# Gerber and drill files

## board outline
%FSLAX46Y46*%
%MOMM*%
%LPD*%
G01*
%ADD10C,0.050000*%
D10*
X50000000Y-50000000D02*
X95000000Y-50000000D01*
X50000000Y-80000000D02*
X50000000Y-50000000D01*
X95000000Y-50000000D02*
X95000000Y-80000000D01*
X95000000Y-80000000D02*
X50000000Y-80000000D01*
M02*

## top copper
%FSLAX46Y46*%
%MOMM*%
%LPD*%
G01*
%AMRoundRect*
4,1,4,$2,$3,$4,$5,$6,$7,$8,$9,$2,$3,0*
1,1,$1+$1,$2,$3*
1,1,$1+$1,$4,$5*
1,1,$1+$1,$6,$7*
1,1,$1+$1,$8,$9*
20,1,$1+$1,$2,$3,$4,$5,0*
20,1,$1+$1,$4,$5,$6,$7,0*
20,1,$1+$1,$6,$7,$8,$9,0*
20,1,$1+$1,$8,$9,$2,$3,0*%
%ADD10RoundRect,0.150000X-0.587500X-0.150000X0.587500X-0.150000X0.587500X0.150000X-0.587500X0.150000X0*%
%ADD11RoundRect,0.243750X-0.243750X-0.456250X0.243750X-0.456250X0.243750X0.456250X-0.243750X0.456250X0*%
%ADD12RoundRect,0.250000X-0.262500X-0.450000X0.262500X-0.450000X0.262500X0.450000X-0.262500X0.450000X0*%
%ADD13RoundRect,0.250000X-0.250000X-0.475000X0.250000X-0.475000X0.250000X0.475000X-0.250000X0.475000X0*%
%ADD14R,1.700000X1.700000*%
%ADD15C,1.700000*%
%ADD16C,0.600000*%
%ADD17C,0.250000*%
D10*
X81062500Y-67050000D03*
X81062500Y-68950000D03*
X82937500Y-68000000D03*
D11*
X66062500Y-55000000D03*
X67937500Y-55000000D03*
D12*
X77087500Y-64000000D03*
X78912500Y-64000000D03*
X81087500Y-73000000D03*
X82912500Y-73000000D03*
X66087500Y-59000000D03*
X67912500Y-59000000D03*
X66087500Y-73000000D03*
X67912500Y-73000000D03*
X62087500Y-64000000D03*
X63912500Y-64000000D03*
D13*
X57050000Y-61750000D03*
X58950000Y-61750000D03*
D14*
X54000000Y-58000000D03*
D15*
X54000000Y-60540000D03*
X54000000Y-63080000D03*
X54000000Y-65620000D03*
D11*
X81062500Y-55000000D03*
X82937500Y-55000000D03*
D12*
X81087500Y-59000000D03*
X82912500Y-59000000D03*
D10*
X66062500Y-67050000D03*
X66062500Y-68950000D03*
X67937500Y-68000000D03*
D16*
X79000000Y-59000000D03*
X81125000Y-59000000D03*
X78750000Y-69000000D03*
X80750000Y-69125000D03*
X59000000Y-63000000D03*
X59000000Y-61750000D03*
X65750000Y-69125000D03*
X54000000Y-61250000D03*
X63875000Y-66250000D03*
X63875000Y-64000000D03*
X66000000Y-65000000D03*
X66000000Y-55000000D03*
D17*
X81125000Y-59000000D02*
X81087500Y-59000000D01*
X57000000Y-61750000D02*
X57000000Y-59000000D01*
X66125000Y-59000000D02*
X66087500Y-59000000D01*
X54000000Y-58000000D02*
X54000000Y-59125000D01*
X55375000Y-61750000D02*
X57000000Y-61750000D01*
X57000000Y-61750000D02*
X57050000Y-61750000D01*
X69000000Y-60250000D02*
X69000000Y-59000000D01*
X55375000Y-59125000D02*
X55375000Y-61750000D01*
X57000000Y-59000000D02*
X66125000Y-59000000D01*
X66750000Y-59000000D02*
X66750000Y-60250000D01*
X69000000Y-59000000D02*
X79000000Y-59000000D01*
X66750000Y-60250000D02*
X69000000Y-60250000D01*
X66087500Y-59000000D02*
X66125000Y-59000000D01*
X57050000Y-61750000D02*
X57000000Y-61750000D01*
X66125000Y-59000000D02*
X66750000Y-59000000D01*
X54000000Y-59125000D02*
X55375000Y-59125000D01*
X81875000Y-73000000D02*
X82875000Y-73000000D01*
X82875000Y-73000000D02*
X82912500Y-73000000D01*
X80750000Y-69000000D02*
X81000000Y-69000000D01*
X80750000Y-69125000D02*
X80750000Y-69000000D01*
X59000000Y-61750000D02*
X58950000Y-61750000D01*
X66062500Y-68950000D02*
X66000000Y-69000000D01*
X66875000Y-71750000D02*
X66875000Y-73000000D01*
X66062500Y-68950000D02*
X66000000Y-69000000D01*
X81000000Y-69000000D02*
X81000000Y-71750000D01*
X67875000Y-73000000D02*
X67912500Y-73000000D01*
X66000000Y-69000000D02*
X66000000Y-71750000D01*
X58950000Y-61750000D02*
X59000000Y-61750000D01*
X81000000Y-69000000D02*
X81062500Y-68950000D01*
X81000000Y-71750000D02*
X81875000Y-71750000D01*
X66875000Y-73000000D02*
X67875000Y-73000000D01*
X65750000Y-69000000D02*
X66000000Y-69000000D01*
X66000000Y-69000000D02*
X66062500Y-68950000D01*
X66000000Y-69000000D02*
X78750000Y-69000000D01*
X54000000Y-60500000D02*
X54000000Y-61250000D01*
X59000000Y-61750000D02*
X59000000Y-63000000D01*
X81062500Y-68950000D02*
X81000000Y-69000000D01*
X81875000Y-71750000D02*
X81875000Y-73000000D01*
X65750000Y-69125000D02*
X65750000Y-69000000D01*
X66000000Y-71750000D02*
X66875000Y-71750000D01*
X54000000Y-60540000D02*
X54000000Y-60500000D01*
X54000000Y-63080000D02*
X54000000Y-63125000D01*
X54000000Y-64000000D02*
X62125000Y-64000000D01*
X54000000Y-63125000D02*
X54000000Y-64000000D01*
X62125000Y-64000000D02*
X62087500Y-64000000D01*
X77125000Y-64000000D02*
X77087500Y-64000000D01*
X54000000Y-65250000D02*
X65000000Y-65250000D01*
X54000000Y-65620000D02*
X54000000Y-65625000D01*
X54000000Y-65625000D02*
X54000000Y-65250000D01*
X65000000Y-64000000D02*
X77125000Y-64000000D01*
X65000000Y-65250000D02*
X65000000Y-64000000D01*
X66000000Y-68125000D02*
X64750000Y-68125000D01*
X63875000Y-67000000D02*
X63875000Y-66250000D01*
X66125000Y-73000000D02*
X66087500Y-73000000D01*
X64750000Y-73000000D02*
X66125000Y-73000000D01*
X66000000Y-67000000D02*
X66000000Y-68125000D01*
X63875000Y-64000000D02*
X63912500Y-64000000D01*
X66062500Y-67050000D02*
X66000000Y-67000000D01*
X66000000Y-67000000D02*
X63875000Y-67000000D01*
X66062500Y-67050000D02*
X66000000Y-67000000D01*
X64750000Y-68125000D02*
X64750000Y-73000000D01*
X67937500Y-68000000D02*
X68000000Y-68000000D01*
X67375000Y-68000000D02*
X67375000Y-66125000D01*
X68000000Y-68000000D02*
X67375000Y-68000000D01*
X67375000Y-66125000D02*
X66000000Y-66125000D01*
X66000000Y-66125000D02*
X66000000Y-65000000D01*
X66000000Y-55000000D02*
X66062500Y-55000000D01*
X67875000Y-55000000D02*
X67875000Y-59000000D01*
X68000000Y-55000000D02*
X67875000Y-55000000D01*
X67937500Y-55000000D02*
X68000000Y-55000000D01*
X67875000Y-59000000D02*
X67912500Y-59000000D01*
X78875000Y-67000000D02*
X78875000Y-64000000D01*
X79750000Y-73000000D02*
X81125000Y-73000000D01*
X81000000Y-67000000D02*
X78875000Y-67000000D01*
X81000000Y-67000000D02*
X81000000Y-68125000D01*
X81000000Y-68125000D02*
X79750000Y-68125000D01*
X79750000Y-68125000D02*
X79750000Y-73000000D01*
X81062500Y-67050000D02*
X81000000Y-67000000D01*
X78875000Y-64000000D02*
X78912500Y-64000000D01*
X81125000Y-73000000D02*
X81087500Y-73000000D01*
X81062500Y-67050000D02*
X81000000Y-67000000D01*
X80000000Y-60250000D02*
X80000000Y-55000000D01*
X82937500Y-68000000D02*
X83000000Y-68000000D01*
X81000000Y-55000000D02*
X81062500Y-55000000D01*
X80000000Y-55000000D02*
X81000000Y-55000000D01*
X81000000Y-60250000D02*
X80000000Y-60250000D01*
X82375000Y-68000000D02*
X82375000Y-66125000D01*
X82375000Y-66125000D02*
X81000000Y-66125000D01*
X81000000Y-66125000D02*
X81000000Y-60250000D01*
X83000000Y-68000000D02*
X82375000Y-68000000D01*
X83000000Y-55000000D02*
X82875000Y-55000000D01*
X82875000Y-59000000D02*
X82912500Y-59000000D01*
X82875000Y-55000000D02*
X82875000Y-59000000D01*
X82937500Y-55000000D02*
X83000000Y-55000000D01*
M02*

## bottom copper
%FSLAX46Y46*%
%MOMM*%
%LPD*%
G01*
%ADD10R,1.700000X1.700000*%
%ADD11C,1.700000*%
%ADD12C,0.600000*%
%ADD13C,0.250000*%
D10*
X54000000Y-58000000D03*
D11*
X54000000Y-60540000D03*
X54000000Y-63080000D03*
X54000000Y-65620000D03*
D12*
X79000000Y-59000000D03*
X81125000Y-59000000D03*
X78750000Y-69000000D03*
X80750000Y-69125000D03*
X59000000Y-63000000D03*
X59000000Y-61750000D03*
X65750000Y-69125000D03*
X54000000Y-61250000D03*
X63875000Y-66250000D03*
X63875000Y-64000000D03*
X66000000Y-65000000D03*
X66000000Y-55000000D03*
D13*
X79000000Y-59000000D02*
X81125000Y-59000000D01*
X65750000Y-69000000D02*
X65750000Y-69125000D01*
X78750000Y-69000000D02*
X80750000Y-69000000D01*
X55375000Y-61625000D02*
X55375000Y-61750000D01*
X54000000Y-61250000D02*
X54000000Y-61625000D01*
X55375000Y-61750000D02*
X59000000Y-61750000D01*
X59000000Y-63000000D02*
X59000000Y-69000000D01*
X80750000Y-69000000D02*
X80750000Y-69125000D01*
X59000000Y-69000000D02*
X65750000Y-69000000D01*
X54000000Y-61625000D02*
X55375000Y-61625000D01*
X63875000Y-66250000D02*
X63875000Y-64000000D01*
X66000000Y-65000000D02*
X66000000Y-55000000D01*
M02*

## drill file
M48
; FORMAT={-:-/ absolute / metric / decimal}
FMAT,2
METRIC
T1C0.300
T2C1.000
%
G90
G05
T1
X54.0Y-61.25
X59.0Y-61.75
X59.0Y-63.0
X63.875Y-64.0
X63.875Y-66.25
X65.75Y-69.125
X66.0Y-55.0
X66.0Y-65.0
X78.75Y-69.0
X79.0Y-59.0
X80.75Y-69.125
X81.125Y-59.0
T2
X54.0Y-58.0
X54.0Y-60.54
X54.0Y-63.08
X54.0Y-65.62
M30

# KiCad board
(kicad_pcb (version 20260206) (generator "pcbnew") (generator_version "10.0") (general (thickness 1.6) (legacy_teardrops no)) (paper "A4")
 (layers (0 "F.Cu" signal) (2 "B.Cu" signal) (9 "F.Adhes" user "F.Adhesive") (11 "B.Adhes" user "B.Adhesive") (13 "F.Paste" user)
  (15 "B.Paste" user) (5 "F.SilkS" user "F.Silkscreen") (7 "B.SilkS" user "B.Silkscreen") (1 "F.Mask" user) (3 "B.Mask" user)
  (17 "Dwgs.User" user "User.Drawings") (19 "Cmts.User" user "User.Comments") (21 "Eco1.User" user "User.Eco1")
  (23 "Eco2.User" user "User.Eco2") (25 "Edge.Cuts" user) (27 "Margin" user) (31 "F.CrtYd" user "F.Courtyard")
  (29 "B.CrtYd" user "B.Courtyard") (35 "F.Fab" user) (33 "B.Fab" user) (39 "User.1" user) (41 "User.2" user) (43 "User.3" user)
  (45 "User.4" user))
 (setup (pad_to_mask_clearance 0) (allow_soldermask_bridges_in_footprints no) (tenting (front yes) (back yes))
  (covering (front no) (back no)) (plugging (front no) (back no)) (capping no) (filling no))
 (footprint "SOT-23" (layer "F.Cu") (at 82 68)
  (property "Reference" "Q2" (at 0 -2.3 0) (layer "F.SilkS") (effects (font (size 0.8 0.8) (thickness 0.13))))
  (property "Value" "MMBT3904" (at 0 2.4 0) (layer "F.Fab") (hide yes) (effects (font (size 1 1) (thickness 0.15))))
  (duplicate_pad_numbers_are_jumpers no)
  (pad "1" smd roundrect (at -0.9375 -0.95) (size 1.475 0.6) (layers "F.Cu" "F.Mask" "F.Paste") (roundrect_rratio 0.25) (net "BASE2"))
  (pad "2" smd roundrect (at -0.9375 0.95) (size 1.475 0.6) (layers "F.Cu" "F.Mask" "F.Paste") (roundrect_rratio 0.25) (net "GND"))
  (pad "3" smd roundrect (at 0.9375 0) (size 1.475 0.6) (layers "F.Cu" "F.Mask" "F.Paste") (roundrect_rratio 0.25) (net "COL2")))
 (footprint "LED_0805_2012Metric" (layer "F.Cu") (at 67 55)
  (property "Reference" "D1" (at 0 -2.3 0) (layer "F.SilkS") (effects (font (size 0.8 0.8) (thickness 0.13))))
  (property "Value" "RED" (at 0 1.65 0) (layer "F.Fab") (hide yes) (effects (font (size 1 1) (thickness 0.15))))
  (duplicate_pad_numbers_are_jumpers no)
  (pad "1" smd roundrect (at -0.9375 0) (size 0.975 1.4) (layers "F.Cu" "F.Mask" "F.Paste") (roundrect_rratio 0.25) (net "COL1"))
  (pad "2" smd roundrect (at 0.9375 0) (size 0.975 1.4) (layers "F.Cu" "F.Mask" "F.Paste") (roundrect_rratio 0.25) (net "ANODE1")))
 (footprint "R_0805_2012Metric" (layer "F.Cu") (at 78 64)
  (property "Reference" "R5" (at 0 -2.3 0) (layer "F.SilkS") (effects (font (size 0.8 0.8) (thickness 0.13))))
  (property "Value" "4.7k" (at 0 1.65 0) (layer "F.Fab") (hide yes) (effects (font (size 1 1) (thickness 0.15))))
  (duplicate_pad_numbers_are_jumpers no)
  (pad "1" smd roundrect (at -0.9125 0) (size 1.025 1.4) (layers "F.Cu" "F.Mask" "F.Paste") (roundrect_rratio 0.243902) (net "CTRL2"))
  (pad "2" smd roundrect (at 0.9125 0) (size 1.025 1.4) (layers "F.Cu" "F.Mask" "F.Paste") (roundrect_rratio 0.243902) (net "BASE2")))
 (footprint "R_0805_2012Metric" (layer "F.Cu") (at 82 73)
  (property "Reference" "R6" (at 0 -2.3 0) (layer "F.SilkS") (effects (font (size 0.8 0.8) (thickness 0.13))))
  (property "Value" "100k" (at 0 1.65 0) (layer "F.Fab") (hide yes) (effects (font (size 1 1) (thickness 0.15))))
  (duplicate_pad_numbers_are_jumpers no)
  (pad "1" smd roundrect (at -0.9125 0) (size 1.025 1.4) (layers "F.Cu" "F.Mask" "F.Paste") (roundrect_rratio 0.243902) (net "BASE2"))
  (pad "2" smd roundrect (at 0.9125 0) (size 1.025 1.4) (layers "F.Cu" "F.Mask" "F.Paste") (roundrect_rratio 0.243902) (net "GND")))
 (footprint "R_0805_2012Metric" (layer "F.Cu") (at 67 59)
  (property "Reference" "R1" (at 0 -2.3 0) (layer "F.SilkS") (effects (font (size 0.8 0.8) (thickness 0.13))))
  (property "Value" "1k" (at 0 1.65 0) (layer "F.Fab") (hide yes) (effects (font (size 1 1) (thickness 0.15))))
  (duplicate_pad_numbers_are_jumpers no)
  (pad "1" smd roundrect (at -0.9125 0) (size 1.025 1.4) (layers "F.Cu" "F.Mask" "F.Paste") (roundrect_rratio 0.243902) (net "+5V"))
  (pad "2" smd roundrect (at 0.9125 0) (size 1.025 1.4) (layers "F.Cu" "F.Mask" "F.Paste") (roundrect_rratio 0.243902) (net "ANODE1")))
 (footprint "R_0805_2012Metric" (layer "F.Cu") (at 67 73)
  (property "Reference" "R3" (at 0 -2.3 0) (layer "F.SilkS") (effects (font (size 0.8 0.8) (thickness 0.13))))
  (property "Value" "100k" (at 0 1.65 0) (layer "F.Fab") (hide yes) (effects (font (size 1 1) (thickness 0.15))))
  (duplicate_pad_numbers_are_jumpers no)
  (pad "1" smd roundrect (at -0.9125 0) (size 1.025 1.4) (layers "F.Cu" "F.Mask" "F.Paste") (roundrect_rratio 0.243902) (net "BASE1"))
  (pad "2" smd roundrect (at 0.9125 0) (size 1.025 1.4) (layers "F.Cu" "F.Mask" "F.Paste") (roundrect_rratio 0.243902) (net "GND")))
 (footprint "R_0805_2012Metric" (layer "F.Cu") (at 63 64)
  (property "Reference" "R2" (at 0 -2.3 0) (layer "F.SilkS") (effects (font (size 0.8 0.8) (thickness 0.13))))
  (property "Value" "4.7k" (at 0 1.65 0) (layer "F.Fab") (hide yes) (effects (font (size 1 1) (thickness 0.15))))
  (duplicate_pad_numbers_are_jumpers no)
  (pad "1" smd roundrect (at -0.9125 0) (size 1.025 1.4) (layers "F.Cu" "F.Mask" "F.Paste") (roundrect_rratio 0.243902) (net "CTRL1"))
  (pad "2" smd roundrect (at 0.9125 0) (size 1.025 1.4) (layers "F.Cu" "F.Mask" "F.Paste") (roundrect_rratio 0.243902) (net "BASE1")))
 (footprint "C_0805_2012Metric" (layer "F.Cu") (at 58 61.75)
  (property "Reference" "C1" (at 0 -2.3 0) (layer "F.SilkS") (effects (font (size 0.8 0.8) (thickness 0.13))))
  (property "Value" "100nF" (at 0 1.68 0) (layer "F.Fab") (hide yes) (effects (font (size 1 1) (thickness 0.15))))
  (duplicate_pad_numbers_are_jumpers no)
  (pad "1" smd roundrect (at -0.95 0) (size 1 1.45) (layers "F.Cu" "F.Mask" "F.Paste") (roundrect_rratio 0.25) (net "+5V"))
  (pad "2" smd roundrect (at 0.95 0) (size 1 1.45) (layers "F.Cu" "F.Mask" "F.Paste") (roundrect_rratio 0.25) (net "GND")))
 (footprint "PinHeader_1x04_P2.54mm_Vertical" (layer "F.Cu") (at 54 58)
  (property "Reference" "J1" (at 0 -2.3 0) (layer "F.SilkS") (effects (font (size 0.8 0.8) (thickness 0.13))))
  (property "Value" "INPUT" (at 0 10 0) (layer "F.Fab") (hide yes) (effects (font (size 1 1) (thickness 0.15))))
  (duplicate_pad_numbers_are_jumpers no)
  (pad "1" thru_hole rect (at 0 0) (size 1.7 1.7) (drill 1) (layers "*.Cu" "*.Mask") (remove_unused_layers no) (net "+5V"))
  (pad "2" thru_hole circle (at 0 2.54) (size 1.7 1.7) (drill 1) (layers "*.Cu" "*.Mask") (remove_unused_layers no) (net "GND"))
  (pad "3" thru_hole circle (at 0 5.08) (size 1.7 1.7) (drill 1) (layers "*.Cu" "*.Mask") (remove_unused_layers no) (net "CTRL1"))
  (pad "4" thru_hole circle (at 0 7.62) (size 1.7 1.7) (drill 1) (layers "*.Cu" "*.Mask") (remove_unused_layers no) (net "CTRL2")))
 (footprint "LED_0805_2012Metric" (layer "F.Cu") (at 82 55)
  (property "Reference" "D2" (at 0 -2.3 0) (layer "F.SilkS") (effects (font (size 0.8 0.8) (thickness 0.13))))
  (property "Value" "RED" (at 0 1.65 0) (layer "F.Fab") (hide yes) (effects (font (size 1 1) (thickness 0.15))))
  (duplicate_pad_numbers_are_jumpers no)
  (pad "1" smd roundrect (at -0.9375 0) (size 0.975 1.4) (layers "F.Cu" "F.Mask" "F.Paste") (roundrect_rratio 0.25) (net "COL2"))
  (pad "2" smd roundrect (at 0.9375 0) (size 0.975 1.4) (layers "F.Cu" "F.Mask" "F.Paste") (roundrect_rratio 0.25) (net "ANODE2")))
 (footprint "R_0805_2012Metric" (layer "F.Cu") (at 82 59)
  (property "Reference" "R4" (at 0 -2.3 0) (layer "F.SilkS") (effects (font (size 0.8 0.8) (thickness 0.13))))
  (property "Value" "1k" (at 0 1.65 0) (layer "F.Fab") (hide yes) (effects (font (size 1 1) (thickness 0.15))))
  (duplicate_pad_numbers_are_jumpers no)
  (pad "1" smd roundrect (at -0.9125 0) (size 1.025 1.4) (layers "F.Cu" "F.Mask" "F.Paste") (roundrect_rratio 0.243902) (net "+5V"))
  (pad "2" smd roundrect (at 0.9125 0) (size 1.025 1.4) (layers "F.Cu" "F.Mask" "F.Paste") (roundrect_rratio 0.243902) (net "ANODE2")))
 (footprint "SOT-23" (layer "F.Cu") (at 67 68)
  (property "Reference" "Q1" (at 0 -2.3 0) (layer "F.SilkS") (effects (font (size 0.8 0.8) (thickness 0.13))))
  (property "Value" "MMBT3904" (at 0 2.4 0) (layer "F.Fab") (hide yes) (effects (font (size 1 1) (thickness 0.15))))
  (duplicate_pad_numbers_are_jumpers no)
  (pad "1" smd roundrect (at -0.9375 -0.95) (size 1.475 0.6) (layers "F.Cu" "F.Mask" "F.Paste") (roundrect_rratio 0.25) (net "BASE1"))
  (pad "2" smd roundrect (at -0.9375 0.95) (size 1.475 0.6) (layers "F.Cu" "F.Mask" "F.Paste") (roundrect_rratio 0.25) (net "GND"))
  (pad "3" smd roundrect (at 0.9375 0) (size 1.475 0.6) (layers "F.Cu" "F.Mask" "F.Paste") (roundrect_rratio 0.25) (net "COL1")))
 (gr_line (start 50 50) (end 95 50) (stroke (width 0.05) (type default)) (layer "Edge.Cuts"))
 (gr_line (start 50 80) (end 50 50) (stroke (width 0.05) (type default)) (layer "Edge.Cuts"))
 (gr_line (start 95 50) (end 95 80) (stroke (width 0.05) (type default)) (layer "Edge.Cuts"))
 (gr_line (start 95 80) (end 50 80) (stroke (width 0.05) (type default)) (layer "Edge.Cuts"))
 (segment (start 81.125 59) (end 81.0875 59) (width 0.25) (layer "F.Cu") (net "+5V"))
 (segment (start 57 61.75) (end 57 59) (width 0.25) (layer "F.Cu") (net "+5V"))
 (segment (start 66.125 59) (end 66.0875 59) (width 0.25) (layer "F.Cu") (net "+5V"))
 (segment (start 54 58) (end 54 59.125) (width 0.25) (layer "F.Cu") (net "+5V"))
 (segment (start 55.375 61.75) (end 57 61.75) (width 0.25) (layer "F.Cu") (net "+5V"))
 (segment (start 57 61.75) (end 57.05 61.75) (width 0.25) (layer "F.Cu") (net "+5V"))
 (segment (start 69 60.25) (end 69 59) (width 0.25) (layer "F.Cu") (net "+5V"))
 (segment (start 55.375 59.125) (end 55.375 61.75) (width 0.25) (layer "F.Cu") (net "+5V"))
 (segment (start 57 59) (end 66.125 59) (width 0.25) (layer "F.Cu") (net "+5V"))
 (segment (start 66.75 59) (end 66.75 60.25) (width 0.25) (layer "F.Cu") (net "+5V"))
 (segment (start 69 59) (end 79 59) (width 0.25) (layer "F.Cu") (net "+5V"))
 (segment (start 66.75 60.25) (end 69 60.25) (width 0.25) (layer "F.Cu") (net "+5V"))
 (segment (start 66.0875 59) (end 66.125 59) (width 0.25) (layer "F.Cu") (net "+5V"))
 (segment (start 57.05 61.75) (end 57 61.75) (width 0.25) (layer "F.Cu") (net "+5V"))
 (segment (start 66.125 59) (end 66.75 59) (width 0.25) (layer "F.Cu") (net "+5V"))
 (segment (start 54 59.125) (end 55.375 59.125) (width 0.25) (layer "F.Cu") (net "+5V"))
 (via (at 79 59) (size 0.6) (drill 0.3) (layers "F.Cu" "B.Cu") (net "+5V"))
 (via (at 81.125 59) (size 0.6) (drill 0.3) (layers "F.Cu" "B.Cu") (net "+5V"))
 (segment (start 79 59) (end 81.125 59) (width 0.25) (layer "B.Cu") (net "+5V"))
 (segment (start 81.875 73) (end 82.875 73) (width 0.25) (layer "F.Cu") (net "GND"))
 (segment (start 82.875 73) (end 82.9125 73) (width 0.25) (layer "F.Cu") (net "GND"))
 (segment (start 80.75 69) (end 81 69) (width 0.25) (layer "F.Cu") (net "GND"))
 (segment (start 80.75 69.125) (end 80.75 69) (width 0.25) (layer "F.Cu") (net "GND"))
 (segment (start 59 61.75) (end 58.95 61.75) (width 0.25) (layer "F.Cu") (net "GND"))
 (segment (start 66.0625 68.95) (end 66 69) (width 0.25) (layer "F.Cu") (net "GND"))
 (segment (start 66.875 71.75) (end 66.875 73) (width 0.25) (layer "F.Cu") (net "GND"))
 (segment (start 66.0625 68.95) (end 66 69) (width 0.25) (layer "F.Cu") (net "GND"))
 (segment (start 81 69) (end 81 71.75) (width 0.25) (layer "F.Cu") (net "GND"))
 (segment (start 67.875 73) (end 67.9125 73) (width 0.25) (layer "F.Cu") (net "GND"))
 (segment (start 66 69) (end 66 71.75) (width 0.25) (layer "F.Cu") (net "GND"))
 (segment (start 58.95 61.75) (end 59 61.75) (width 0.25) (layer "F.Cu") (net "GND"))
 (segment (start 81 69) (end 81.0625 68.95) (width 0.25) (layer "F.Cu") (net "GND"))
 (segment (start 81 71.75) (end 81.875 71.75) (width 0.25) (layer "F.Cu") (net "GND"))
 (segment (start 66.875 73) (end 67.875 73) (width 0.25) (layer "F.Cu") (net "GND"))
 (segment (start 65.75 69) (end 66 69) (width 0.25) (layer "F.Cu") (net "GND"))
 (segment (start 66 69) (end 66.0625 68.95) (width 0.25) (layer "F.Cu") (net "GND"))
 (segment (start 66 69) (end 78.75 69) (width 0.25) (layer "F.Cu") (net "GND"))
 (segment (start 54 60.5) (end 54 61.25) (width 0.25) (layer "F.Cu") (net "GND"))
 (segment (start 59 61.75) (end 59 63) (width 0.25) (layer "F.Cu") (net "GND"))
 (segment (start 81.0625 68.95) (end 81 69) (width 0.25) (layer "F.Cu") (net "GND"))
 (segment (start 81.875 71.75) (end 81.875 73) (width 0.25) (layer "F.Cu") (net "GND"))
 (segment (start 65.75 69.125) (end 65.75 69) (width 0.25) (layer "F.Cu") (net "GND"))
 (segment (start 66 71.75) (end 66.875 71.75) (width 0.25) (layer "F.Cu") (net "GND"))
 (segment (start 54 60.54) (end 54 60.5) (width 0.25) (layer "F.Cu") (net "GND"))
 (via (at 78.75 69) (size 0.6) (drill 0.3) (layers "F.Cu" "B.Cu") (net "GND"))
 (via (at 80.75 69.125) (size 0.6) (drill 0.3) (layers "F.Cu" "B.Cu") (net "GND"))
 (via (at 59 63) (size 0.6) (drill 0.3) (layers "F.Cu" "B.Cu") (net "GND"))
 (via (at 59 61.75) (size 0.6) (drill 0.3) (layers "F.Cu" "B.Cu") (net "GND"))
 (via (at 65.75 69.125) (size 0.6) (drill 0.3) (layers "F.Cu" "B.Cu") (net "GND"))
 (via (at 54 61.25) (size 0.6) (drill 0.3) (layers "F.Cu" "B.Cu") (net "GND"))
 (segment (start 65.75 69) (end 65.75 69.125) (width 0.25) (layer "B.Cu") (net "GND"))
 (segment (start 78.75 69) (end 80.75 69) (width 0.25) (layer "B.Cu") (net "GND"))
 (segment (start 55.375 61.625) (end 55.375 61.75) (width 0.25) (layer "B.Cu") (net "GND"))
 (segment (start 54 61.25) (end 54 61.625) (width 0.25) (layer "B.Cu") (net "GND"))
 (segment (start 55.375 61.75) (end 59 61.75) (width 0.25) (layer "B.Cu") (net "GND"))
 (segment (start 59 63) (end 59 69) (width 0.25) (layer "B.Cu") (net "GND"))
 (segment (start 80.75 69) (end 80.75 69.125) (width 0.25) (layer "B.Cu") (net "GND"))
 (segment (start 59 69) (end 65.75 69) (width 0.25) (layer "B.Cu") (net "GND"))
 (segment (start 54 61.625) (end 55.375 61.625) (width 0.25) (layer "B.Cu") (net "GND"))
 (segment (start 54 63.08) (end 54 63.125) (width 0.25) (layer "F.Cu") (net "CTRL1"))
 (segment (start 54 64) (end 62.125 64) (width 0.25) (layer "F.Cu") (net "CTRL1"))
 (segment (start 54 63.125) (end 54 64) (width 0.25) (layer "F.Cu") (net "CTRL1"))
 (segment (start 62.125 64) (end 62.0875 64) (width 0.25) (layer "F.Cu") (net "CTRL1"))
 (segment (start 77.125 64) (end 77.0875 64) (width 0.25) (layer "F.Cu") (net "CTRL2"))
 (segment (start 54 65.25) (end 65 65.25) (width 0.25) (layer "F.Cu") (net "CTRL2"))
 (segment (start 54 65.62) (end 54 65.625) (width 0.25) (layer "F.Cu") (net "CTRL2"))
 (segment (start 54 65.625) (end 54 65.25) (width 0.25) (layer "F.Cu") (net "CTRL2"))
 (segment (start 65 64) (end 77.125 64) (width 0.25) (layer "F.Cu") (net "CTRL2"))
 (segment (start 65 65.25) (end 65 64) (width 0.25) (layer "F.Cu") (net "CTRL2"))
 (segment (start 66 68.125) (end 64.75 68.125) (width 0.25) (layer "F.Cu") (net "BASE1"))
 (segment (start 63.875 67) (end 63.875 66.25) (width 0.25) (layer "F.Cu") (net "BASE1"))
 (segment (start 66.125 73) (end 66.0875 73) (width 0.25) (layer "F.Cu") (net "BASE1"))
 (segment (start 64.75 73) (end 66.125 73) (width 0.25) (layer "F.Cu") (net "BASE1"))
 (segment (start 66 67) (end 66 68.125) (width 0.25) (layer "F.Cu") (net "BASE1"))
 (segment (start 63.875 64) (end 63.9125 64) (width 0.25) (layer "F.Cu") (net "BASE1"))
 (segment (start 66.0625 67.05) (end 66 67) (width 0.25) (layer "F.Cu") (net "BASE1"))
 (segment (start 66 67) (end 63.875 67) (width 0.25) (layer "F.Cu") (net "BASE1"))
 (segment (start 66.0625 67.05) (end 66 67) (width 0.25) (layer "F.Cu") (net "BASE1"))
 (segment (start 64.75 68.125) (end 64.75 73) (width 0.25) (layer "F.Cu") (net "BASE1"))
 (via (at 63.875 66.25) (size 0.6) (drill 0.3) (layers "F.Cu" "B.Cu") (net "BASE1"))
 (via (at 63.875 64) (size 0.6) (drill 0.3) (layers "F.Cu" "B.Cu") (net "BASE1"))
 (segment (start 63.875 66.25) (end 63.875 64) (width 0.25) (layer "B.Cu") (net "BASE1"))
 (segment (start 67.9375 68) (end 68 68) (width 0.25) (layer "F.Cu") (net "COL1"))
 (segment (start 67.375 68) (end 67.375 66.125) (width 0.25) (layer "F.Cu") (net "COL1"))
 (segment (start 68 68) (end 67.375 68) (width 0.25) (layer "F.Cu") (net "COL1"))
 (segment (start 67.375 66.125) (end 66 66.125) (width 0.25) (layer "F.Cu") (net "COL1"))
 (segment (start 66 66.125) (end 66 65) (width 0.25) (layer "F.Cu") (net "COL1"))
 (segment (start 66 55) (end 66.0625 55) (width 0.25) (layer "F.Cu") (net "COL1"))
 (via (at 66 65) (size 0.6) (drill 0.3) (layers "F.Cu" "B.Cu") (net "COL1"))
 (via (at 66 55) (size 0.6) (drill 0.3) (layers "F.Cu" "B.Cu") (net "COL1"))
 (segment (start 66 65) (end 66 55) (width 0.25) (layer "B.Cu") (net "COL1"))
 (segment (start 67.875 55) (end 67.875 59) (width 0.25) (layer "F.Cu") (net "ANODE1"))
 (segment (start 68 55) (end 67.875 55) (width 0.25) (layer "F.Cu") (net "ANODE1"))
 (segment (start 67.9375 55) (end 68 55) (width 0.25) (layer "F.Cu") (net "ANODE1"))
 (segment (start 67.875 59) (end 67.9125 59) (width 0.25) (layer "F.Cu") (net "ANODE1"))
 (segment (start 78.875 67) (end 78.875 64) (width 0.25) (layer "F.Cu") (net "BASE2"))
 (segment (start 79.75 73) (end 81.125 73) (width 0.25) (layer "F.Cu") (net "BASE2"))
 (segment (start 81 67) (end 78.875 67) (width 0.25) (layer "F.Cu") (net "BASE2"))
 (segment (start 81 67) (end 81 68.125) (width 0.25) (layer "F.Cu") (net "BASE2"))
 (segment (start 81 68.125) (end 79.75 68.125) (width 0.25) (layer "F.Cu") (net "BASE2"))
 (segment (start 79.75 68.125) (end 79.75 73) (width 0.25) (layer "F.Cu") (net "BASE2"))
 (segment (start 81.0625 67.05) (end 81 67) (width 0.25) (layer "F.Cu") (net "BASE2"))
 (segment (start 78.875 64) (end 78.9125 64) (width 0.25) (layer "F.Cu") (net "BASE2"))
 (segment (start 81.125 73) (end 81.0875 73) (width 0.25) (layer "F.Cu") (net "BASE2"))
 (segment (start 81.0625 67.05) (end 81 67) (width 0.25) (layer "F.Cu") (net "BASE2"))
 (segment (start 80 60.25) (end 80 55) (width 0.25) (layer "F.Cu") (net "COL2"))
 (segment (start 82.9375 68) (end 83 68) (width 0.25) (layer "F.Cu") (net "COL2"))
 (segment (start 81 55) (end 81.0625 55) (width 0.25) (layer "F.Cu") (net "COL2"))
 (segment (start 80 55) (end 81 55) (width 0.25) (layer "F.Cu") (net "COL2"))
 (segment (start 81 60.25) (end 80 60.25) (width 0.25) (layer "F.Cu") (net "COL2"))
 (segment (start 82.375 68) (end 82.375 66.125) (width 0.25) (layer "F.Cu") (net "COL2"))
 (segment (start 82.375 66.125) (end 81 66.125) (width 0.25) (layer "F.Cu") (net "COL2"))
 (segment (start 81 66.125) (end 81 60.25) (width 0.25) (layer "F.Cu") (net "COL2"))
 (segment (start 83 68) (end 82.375 68) (width 0.25) (layer "F.Cu") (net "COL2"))
 (segment (start 83 55) (end 82.875 55) (width 0.25) (layer "F.Cu") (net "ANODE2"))
 (segment (start 82.875 59) (end 82.9125 59) (width 0.25) (layer "F.Cu") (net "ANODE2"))
 (segment (start 82.875 55) (end 82.875 59) (width 0.25) (layer "F.Cu") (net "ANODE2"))
 (segment (start 82.9375 55) (end 83 55) (width 0.25) (layer "F.Cu") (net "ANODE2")))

